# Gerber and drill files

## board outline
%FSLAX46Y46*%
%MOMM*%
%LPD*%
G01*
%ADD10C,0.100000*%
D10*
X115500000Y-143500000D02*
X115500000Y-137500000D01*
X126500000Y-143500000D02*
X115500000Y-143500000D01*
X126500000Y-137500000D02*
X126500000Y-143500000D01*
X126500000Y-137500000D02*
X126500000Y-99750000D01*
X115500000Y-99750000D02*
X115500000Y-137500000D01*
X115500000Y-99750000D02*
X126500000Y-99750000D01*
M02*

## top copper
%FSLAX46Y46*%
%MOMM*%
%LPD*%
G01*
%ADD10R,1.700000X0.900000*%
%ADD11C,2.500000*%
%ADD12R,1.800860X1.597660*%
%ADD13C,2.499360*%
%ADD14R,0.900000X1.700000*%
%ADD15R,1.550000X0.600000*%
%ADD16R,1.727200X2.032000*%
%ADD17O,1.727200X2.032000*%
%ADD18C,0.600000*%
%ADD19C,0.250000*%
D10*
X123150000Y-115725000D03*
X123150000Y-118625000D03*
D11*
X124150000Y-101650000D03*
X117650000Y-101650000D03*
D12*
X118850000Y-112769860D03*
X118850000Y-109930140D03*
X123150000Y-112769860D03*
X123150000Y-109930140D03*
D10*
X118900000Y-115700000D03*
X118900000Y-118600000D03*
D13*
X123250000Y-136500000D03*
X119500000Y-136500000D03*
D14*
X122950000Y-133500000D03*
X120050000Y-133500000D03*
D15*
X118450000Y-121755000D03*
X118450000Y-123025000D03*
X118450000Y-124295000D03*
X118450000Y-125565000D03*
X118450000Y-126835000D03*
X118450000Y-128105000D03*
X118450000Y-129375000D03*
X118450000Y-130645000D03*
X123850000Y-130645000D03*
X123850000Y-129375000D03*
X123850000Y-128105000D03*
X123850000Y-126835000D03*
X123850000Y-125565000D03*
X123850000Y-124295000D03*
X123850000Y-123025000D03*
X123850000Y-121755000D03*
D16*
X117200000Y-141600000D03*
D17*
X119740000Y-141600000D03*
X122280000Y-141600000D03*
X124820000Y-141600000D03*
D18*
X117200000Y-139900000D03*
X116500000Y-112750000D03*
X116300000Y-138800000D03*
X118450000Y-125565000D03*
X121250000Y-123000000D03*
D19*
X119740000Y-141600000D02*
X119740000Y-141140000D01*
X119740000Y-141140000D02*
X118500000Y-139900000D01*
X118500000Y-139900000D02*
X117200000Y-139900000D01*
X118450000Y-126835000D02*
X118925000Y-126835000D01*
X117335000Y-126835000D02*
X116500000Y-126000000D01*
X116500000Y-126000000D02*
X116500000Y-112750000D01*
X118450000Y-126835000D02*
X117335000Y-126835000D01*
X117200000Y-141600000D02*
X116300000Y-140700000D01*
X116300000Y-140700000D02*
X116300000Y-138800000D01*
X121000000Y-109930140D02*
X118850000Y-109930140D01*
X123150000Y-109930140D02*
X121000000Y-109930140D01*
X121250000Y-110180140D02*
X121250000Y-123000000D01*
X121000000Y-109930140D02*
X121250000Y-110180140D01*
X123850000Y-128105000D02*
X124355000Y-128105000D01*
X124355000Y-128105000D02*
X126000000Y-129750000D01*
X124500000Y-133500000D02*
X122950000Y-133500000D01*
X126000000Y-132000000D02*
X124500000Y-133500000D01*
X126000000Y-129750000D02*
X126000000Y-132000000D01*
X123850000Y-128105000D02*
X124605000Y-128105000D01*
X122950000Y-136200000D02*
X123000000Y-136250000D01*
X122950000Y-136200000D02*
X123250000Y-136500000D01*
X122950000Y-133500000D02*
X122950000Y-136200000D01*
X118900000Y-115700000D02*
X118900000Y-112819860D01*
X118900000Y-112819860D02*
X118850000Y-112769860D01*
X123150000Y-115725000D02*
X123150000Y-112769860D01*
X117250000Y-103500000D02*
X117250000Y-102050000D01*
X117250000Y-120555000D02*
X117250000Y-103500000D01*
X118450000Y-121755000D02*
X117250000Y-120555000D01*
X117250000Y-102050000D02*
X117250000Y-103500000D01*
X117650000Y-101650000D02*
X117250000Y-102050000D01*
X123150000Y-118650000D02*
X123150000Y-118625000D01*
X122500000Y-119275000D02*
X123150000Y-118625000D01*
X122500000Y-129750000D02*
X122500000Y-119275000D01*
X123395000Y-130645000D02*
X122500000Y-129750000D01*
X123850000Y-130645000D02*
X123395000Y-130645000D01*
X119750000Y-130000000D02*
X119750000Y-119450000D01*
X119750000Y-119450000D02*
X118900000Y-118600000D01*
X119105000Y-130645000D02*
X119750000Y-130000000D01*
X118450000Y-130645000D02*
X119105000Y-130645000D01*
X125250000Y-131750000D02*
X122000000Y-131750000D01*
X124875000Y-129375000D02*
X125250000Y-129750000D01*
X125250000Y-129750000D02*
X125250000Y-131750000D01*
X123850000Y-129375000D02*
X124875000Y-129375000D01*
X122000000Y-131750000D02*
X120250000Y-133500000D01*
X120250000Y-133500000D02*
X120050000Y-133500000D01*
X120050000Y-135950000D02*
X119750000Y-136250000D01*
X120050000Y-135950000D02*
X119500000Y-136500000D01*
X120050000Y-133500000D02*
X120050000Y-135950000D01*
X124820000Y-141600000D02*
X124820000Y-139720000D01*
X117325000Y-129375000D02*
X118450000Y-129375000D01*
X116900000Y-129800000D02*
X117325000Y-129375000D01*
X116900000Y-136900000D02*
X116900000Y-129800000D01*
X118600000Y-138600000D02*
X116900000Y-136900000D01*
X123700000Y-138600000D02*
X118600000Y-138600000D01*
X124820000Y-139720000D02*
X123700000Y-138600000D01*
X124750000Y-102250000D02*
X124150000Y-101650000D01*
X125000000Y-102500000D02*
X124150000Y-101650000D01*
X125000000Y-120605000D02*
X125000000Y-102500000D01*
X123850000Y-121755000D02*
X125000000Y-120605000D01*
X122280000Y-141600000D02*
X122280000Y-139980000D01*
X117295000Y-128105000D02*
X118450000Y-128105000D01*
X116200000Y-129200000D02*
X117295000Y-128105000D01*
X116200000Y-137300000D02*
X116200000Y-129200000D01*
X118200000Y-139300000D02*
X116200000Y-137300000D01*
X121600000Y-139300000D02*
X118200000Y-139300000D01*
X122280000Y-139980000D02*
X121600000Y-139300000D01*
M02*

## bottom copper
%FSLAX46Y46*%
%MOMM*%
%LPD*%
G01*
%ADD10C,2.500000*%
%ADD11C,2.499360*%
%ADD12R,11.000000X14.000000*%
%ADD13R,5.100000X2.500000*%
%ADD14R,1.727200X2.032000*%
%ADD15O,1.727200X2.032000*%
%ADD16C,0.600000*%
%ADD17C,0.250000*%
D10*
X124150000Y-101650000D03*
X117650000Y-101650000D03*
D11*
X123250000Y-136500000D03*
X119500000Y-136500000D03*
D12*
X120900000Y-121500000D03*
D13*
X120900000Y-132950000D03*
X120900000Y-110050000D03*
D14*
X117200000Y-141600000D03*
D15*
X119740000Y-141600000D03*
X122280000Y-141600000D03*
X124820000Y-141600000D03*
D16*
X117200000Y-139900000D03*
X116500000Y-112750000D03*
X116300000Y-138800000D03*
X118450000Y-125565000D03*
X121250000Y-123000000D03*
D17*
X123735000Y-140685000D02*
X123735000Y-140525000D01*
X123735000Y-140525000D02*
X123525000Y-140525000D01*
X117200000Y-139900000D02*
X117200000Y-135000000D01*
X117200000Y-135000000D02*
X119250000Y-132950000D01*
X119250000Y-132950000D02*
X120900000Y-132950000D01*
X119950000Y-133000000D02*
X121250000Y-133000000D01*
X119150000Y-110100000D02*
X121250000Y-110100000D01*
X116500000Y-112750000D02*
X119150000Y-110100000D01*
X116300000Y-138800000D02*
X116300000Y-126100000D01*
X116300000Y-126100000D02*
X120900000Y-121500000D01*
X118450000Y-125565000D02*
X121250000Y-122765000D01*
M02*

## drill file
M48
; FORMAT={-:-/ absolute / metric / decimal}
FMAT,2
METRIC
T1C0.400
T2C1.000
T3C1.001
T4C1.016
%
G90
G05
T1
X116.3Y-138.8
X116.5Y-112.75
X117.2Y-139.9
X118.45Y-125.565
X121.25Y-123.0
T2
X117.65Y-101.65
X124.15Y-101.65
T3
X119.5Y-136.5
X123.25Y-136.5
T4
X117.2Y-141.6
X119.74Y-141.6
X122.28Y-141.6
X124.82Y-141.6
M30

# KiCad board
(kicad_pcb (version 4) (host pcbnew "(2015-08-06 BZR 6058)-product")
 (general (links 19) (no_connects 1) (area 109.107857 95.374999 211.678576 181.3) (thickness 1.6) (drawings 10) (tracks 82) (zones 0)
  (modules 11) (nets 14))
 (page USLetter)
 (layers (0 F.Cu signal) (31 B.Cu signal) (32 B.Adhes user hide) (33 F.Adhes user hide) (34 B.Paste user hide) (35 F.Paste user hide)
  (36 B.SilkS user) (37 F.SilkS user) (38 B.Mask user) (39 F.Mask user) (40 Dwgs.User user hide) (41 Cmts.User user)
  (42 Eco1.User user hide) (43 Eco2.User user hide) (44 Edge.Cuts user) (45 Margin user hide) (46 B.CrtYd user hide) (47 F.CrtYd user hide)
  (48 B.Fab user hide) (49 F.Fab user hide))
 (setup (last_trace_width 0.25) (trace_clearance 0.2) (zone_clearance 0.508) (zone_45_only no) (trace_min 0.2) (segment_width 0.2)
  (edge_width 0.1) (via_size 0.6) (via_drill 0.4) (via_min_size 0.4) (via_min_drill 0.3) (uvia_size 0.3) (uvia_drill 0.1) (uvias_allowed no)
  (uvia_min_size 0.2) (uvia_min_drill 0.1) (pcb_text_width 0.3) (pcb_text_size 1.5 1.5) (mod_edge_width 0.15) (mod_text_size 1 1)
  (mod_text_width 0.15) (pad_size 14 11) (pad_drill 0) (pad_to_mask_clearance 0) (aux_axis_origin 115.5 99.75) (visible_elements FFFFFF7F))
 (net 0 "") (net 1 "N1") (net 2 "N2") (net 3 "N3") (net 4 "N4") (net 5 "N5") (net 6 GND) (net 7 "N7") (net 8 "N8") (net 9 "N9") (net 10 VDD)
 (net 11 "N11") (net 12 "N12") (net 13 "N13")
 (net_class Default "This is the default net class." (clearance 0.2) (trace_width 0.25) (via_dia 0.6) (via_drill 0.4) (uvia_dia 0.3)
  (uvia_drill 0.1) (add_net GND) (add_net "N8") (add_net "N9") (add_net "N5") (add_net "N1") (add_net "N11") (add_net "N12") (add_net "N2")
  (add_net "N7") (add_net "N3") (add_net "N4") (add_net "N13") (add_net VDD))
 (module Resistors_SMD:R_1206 (layer F.Cu) (at 123.15 117.175 270)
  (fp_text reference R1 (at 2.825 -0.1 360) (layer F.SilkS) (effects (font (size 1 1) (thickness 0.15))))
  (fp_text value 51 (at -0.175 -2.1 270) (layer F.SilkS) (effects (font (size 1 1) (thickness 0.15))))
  (pad 1 smd rect (at -1.45 0 270) (size 0.9 1.7) (layers F.Cu F.Paste F.Mask) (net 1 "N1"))
  (pad 2 smd rect (at 1.45 0 270) (size 0.9 1.7) (layers F.Cu F.Paste F.Mask) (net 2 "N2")))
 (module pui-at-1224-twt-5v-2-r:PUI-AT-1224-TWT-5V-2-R (layer F.Cu) (at 120.9 101.65 180)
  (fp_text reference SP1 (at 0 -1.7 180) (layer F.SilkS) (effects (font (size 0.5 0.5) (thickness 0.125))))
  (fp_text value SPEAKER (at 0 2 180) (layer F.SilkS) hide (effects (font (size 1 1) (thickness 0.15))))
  (pad 1 thru_hole circle (at -3.25 0 180) (size 2.5 2.5) (drill 1) (layers *.Cu *.Mask F.SilkS) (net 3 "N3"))
  (pad 2 thru_hole circle (at 3.25 0 180) (size 2.5 2.5) (drill 1) (layers *.Cu *.Mask F.SilkS) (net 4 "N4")))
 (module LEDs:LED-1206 (layer F.Cu) (at 118.85 111.35 270)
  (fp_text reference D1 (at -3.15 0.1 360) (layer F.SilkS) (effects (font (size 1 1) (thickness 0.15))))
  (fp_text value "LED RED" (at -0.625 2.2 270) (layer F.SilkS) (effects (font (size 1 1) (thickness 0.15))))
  (pad 2 smd rect (at 1.41986 0 90) (size 1.59766 1.80086) (layers F.Cu F.Paste F.Mask) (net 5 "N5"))
  (pad 1 smd rect (at -1.41986 0 90) (size 1.59766 1.80086) (layers F.Cu F.Paste F.Mask) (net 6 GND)))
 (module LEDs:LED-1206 (layer F.Cu) (at 123.15 111.35 270)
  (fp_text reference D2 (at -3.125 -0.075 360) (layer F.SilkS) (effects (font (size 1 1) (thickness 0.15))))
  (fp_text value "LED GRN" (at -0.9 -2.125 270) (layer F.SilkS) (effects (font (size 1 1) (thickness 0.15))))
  (pad 2 smd rect (at 1.41986 0 90) (size 1.59766 1.80086) (layers F.Cu F.Paste F.Mask) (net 1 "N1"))
  (pad 1 smd rect (at -1.41986 0 90) (size 1.59766 1.80086) (layers F.Cu F.Paste F.Mask) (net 6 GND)))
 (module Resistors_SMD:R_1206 (layer F.Cu) (at 118.9 117.15 270)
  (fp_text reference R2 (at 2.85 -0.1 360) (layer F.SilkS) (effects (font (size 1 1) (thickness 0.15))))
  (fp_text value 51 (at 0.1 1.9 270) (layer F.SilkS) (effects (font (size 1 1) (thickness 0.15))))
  (pad 1 smd rect (at -1.45 0 270) (size 0.9 1.7) (layers F.Cu F.Paste F.Mask) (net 5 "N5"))
  (pad 2 smd rect (at 1.45 0 270) (size 0.9 1.7) (layers F.Cu F.Paste F.Mask) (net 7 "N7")))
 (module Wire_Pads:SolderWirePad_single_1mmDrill (layer F.Cu) (at 123.25 136.5)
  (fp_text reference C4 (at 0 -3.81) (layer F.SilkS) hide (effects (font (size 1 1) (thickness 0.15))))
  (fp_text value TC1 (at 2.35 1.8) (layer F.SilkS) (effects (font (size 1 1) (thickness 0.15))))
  (pad 1 thru_hole circle (at 0 0) (size 2.49936 2.49936) (drill 1.00076) (layers *.Cu *.Mask F.SilkS) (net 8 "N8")))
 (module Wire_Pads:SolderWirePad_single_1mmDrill (layer F.Cu) (at 119.5 136.5)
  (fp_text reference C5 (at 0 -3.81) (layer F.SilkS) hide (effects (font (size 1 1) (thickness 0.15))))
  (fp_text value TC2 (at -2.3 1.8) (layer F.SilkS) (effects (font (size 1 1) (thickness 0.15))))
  (pad 1 thru_hole circle (at 0 0) (size 2.49936 2.49936) (drill 1.00076) (layers *.Cu *.Mask F.SilkS) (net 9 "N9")))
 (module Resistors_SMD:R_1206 (layer F.Cu) (at 121.5 133.5 180)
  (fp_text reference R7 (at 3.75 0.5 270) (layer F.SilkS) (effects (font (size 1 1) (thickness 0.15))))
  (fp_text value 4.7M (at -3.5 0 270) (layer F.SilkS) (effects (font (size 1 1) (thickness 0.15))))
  (pad 1 smd rect (at -1.45 0 180) (size 0.9 1.7) (layers F.Cu F.Paste F.Mask) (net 8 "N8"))
  (pad 2 smd rect (at 1.45 0 180) (size 0.9 1.7) (layers F.Cu F.Paste F.Mask) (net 9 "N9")))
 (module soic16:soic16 (layer F.Cu) (at 121.15 126.2) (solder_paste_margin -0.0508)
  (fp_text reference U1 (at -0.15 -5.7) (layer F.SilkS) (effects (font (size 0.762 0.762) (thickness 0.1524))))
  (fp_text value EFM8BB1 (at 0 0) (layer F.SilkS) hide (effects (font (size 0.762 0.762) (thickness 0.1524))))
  (pad 1 smd rect (at -2.7 -4.445) (size 1.55 0.6) (layers F.Cu F.Paste F.Mask) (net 4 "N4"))
  (pad 2 smd rect (at -2.7 -3.175) (size 1.55 0.6) (layers F.Cu F.Paste F.Mask))
  (pad 3 smd rect (at -2.7 -1.905) (size 1.55 0.6) (layers F.Cu F.Paste F.Mask))
  (pad 4 smd rect (at -2.7 -0.635) (size 1.55 0.6) (layers F.Cu F.Paste F.Mask) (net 6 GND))
  (pad 5 smd rect (at -2.7 0.635) (size 1.55 0.6) (layers F.Cu F.Paste F.Mask) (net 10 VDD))
  (pad 6 smd rect (at -2.7 1.905) (size 1.55 0.6) (layers F.Cu F.Paste F.Mask) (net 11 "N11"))
  (pad 7 smd rect (at -2.7 3.175) (size 1.55 0.6) (layers F.Cu F.Paste F.Mask) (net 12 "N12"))
  (pad 8 smd rect (at -2.7 4.445) (size 1.55 0.6) (layers F.Cu F.Paste F.Mask) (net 7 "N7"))
  (pad 9 smd rect (at 2.7 4.445) (size 1.55 0.6) (layers F.Cu F.Paste F.Mask) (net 2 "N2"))
  (pad 10 smd rect (at 2.7 3.175) (size 1.55 0.6) (layers F.Cu F.Paste F.Mask) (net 9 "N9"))
  (pad 11 smd rect (at 2.7 1.905) (size 1.55 0.6) (layers F.Cu F.Paste F.Mask) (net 8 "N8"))
  (pad 12 smd rect (at 2.7 0.635) (size 1.55 0.6) (layers F.Cu F.Paste F.Mask))
  (pad 13 smd rect (at 2.7 -0.635) (size 1.55 0.6) (layers F.Cu F.Paste F.Mask) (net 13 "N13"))
  (pad 14 smd rect (at 2.7 -1.905) (size 1.55 0.6) (layers F.Cu F.Paste F.Mask))
  (pad 15 smd rect (at 2.7 -3.175) (size 1.55 0.6) (layers F.Cu F.Paste F.Mask))
  (pad 16 smd rect (at 2.7 -4.445) (size 1.55 0.6) (layers F.Cu F.Paste F.Mask) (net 3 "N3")))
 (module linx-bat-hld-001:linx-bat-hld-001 (layer B.Cu) (at 120.9 121.5 90)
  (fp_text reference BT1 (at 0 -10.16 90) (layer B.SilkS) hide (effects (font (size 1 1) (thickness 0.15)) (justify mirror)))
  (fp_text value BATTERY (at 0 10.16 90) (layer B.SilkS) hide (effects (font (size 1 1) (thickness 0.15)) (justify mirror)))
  (pad 2 smd rect (at 0 0 90) (size 14 11) (layers B.Cu B.Paste B.Mask) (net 6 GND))
  (pad 1 smd rect (at -11.45 0 90) (size 2.5 5.1) (layers B.Cu B.Paste B.Mask) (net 10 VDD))
  (pad 1 smd rect (at 11.45 0 90) (size 2.5 5.1) (layers B.Cu B.Paste B.Mask) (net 10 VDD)))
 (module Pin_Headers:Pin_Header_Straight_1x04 (layer F.Cu) (at 117.2 141.6 90)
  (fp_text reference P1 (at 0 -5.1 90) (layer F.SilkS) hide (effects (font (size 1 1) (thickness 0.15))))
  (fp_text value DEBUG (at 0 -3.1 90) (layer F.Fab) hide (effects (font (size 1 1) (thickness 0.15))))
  (pad 1 thru_hole rect (at 0 0 90) (size 2.032 1.7272) (drill 1.016) (layers *.Cu *.Mask F.SilkS) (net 6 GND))
  (pad 2 thru_hole oval (at 0 2.54 90) (size 2.032 1.7272) (drill 1.016) (layers *.Cu *.Mask F.SilkS) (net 10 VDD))
  (pad 3 thru_hole oval (at 0 5.08 90) (size 2.032 1.7272) (drill 1.016) (layers *.Cu *.Mask F.SilkS) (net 11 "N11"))
  (pad 4 thru_hole oval (at 0 7.62 90) (size 2.032 1.7272) (drill 1.016) (layers *.Cu *.Mask F.SilkS) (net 12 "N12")))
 (gr_line (start 115.5 143.5) (end 115.5 137.5) (angle 90) (layer Edge.Cuts) (width 0.1))
 (gr_line (start 126.5 143.5) (end 115.5 143.5) (angle 90) (layer Edge.Cuts) (width 0.1))
 (gr_line (start 126.5 137.5) (end 126.5 143.5) (angle 90) (layer Edge.Cuts) (width 0.1))
 (gr_line (start 126.5 137.5) (end 126.5 99.75) (angle 90) (layer Edge.Cuts) (width 0.1))
 (gr_line (start 115.5 99.75) (end 115.5 137.5) (angle 90) (layer Edge.Cuts) (width 0.1))
 (gr_line (start 115.5 99.75) (end 126.5 99.75) (angle 90) (layer Edge.Cuts) (width 0.1))
 (segment (start 123.735 140.685) (end 123.735 140.525) (width 0.25) (layer B.Cu) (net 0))
 (segment (start 123.735 140.525) (end 123.525 140.525) (width 0.25) (layer B.Cu) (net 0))
 (segment (start 119.74 141.6) (end 119.74 141.14) (width 0.25) (layer F.Cu) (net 10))
 (segment (start 119.74 141.14) (end 118.5 139.9) (width 0.25) (layer F.Cu) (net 10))
 (segment (start 118.5 139.9) (end 117.2 139.9) (width 0.25) (layer F.Cu) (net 10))
 (via (at 117.2 139.9) (size 0.6) (drill 0.4) (layers F.Cu B.Cu) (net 10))
 (segment (start 117.2 139.9) (end 117.2 135) (width 0.25) (layer B.Cu) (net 10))
 (segment (start 117.2 135) (end 119.25 132.95) (width 0.25) (layer B.Cu) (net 10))
 (segment (start 119.25 132.95) (end 120.9 132.95) (width 0.25) (layer B.Cu) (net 10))
 (segment (start 119.95 133) (end 121.25 133) (width 0.25) (layer B.Cu) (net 10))
 (segment (start 118.45 126.835) (end 118.925 126.835) (width 0.25) (layer F.Cu) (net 10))
 (segment (start 119.15 110.1) (end 121.25 110.1) (width 0.25) (layer B.Cu) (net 10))
 (segment (start 117.335 126.835) (end 116.5 126) (width 0.25) (layer F.Cu) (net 10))
 (segment (start 116.5 126) (end 116.5 112.75) (width 0.25) (layer F.Cu) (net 10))
 (via (at 116.5 112.75) (size 0.6) (layers F.Cu B.Cu) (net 10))
 (segment (start 116.5 112.75) (end 119.15 110.1) (width 0.25) (layer B.Cu) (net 10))
 (segment (start 118.45 126.835) (end 117.335 126.835) (width 0.25) (layer F.Cu) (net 10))
 (segment (start 117.2 141.6) (end 116.3 140.7) (width 0.25) (layer F.Cu) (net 6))
 (segment (start 116.3 138.8) (end 116.3 126.1) (width 0.25) (layer B.Cu) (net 6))
 (via (at 116.3 138.8) (size 0.6) (drill 0.4) (layers F.Cu B.Cu) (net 6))
 (segment (start 116.3 140.7) (end 116.3 138.8) (width 0.25) (layer F.Cu) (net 6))
 (segment (start 116.3 126.1) (end 120.9 121.5) (width 0.25) (layer B.Cu) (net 6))
 (segment (start 118.45 125.565) (end 121.25 122.765) (width 0.25) (layer B.Cu) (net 6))
 (via (at 118.45 125.565) (size 0.6) (layers F.Cu B.Cu) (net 6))
 (segment (start 121 109.93014) (end 118.85 109.93014) (width 0.25) (layer F.Cu) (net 6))
 (segment (start 123.15 109.93014) (end 121 109.93014) (width 0.25) (layer F.Cu) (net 6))
 (segment (start 121.25 110.18014) (end 121.25 123) (width 0.25) (layer F.Cu) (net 6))
 (via (at 121.25 123) (size 0.6) (layers F.Cu B.Cu) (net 6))
 (segment (start 121 109.93014) (end 121.25 110.18014) (width 0.25) (layer F.Cu) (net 6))
 (segment (start 123.85 128.105) (end 124.355 128.105) (width 0.25) (layer F.Cu) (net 8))
 (segment (start 124.355 128.105) (end 126 129.75) (width 0.25) (layer F.Cu) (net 8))
 (segment (start 124.5 133.5) (end 122.95 133.5) (width 0.25) (layer F.Cu) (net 8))
 (segment (start 126 132) (end 124.5 133.5) (width 0.25) (layer F.Cu) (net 8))
 (segment (start 126 129.75) (end 126 132) (width 0.25) (layer F.Cu) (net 8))
 (segment (start 123.85 128.105) (end 124.605 128.105) (width 0.25) (layer F.Cu) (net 8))
 (segment (start 122.95 136.2) (end 123 136.25) (width 0.25) (layer F.Cu) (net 8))
 (segment (start 122.95 136.2) (end 123.25 136.5) (width 0.25) (layer F.Cu) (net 8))
 (segment (start 122.95 133.5) (end 122.95 136.2) (width 0.25) (layer F.Cu) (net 8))
 (segment (start 118.9 115.7) (end 118.9 112.81986) (width 0.25) (layer F.Cu) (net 5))
 (segment (start 118.9 112.81986) (end 118.85 112.76986) (width 0.25) (layer F.Cu) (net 5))
 (segment (start 123.15 115.725) (end 123.15 112.76986) (width 0.25) (layer F.Cu) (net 1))
 (segment (start 117.25 103.5) (end 117.25 102.05) (width 0.25) (layer F.Cu) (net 4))
 (segment (start 117.25 120.555) (end 117.25 103.5) (width 0.25) (layer F.Cu) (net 4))
 (segment (start 118.45 121.755) (end 117.25 120.555) (width 0.25) (layer F.Cu) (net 4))
 (segment (start 117.25 102.05) (end 117.25 103.5) (width 0.25) (layer F.Cu) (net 4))
 (segment (start 117.65 101.65) (end 117.25 102.05) (width 0.25) (layer F.Cu) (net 4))
 (segment (start 123.15 118.65) (end 123.15 118.625) (width 0.25) (layer F.Cu) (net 2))
 (segment (start 122.5 119.275) (end 123.15 118.625) (width 0.25) (layer F.Cu) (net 2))
 (segment (start 122.5 129.75) (end 122.5 119.275) (width 0.25) (layer F.Cu) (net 2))
 (segment (start 123.395 130.645) (end 122.5 129.75) (width 0.25) (layer F.Cu) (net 2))
 (segment (start 123.85 130.645) (end 123.395 130.645) (width 0.25) (layer F.Cu) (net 2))
 (segment (start 119.75 130) (end 119.75 119.45) (width 0.25) (layer F.Cu) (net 7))
 (segment (start 119.75 119.45) (end 118.9 118.6) (width 0.25) (layer F.Cu) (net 7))
 (segment (start 119.105 130.645) (end 119.75 130) (width 0.25) (layer F.Cu) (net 7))
 (segment (start 118.45 130.645) (end 119.105 130.645) (width 0.25) (layer F.Cu) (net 7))
 (segment (start 125.25 131.75) (end 122 131.75) (width 0.25) (layer F.Cu) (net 9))
 (segment (start 124.875 129.375) (end 125.25 129.75) (width 0.25) (layer F.Cu) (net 9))
 (segment (start 125.25 129.75) (end 125.25 131.75) (width 0.25) (layer F.Cu) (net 9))
 (segment (start 123.85 129.375) (end 124.875 129.375) (width 0.25) (layer F.Cu) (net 9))
 (segment (start 122 131.75) (end 120.25 133.5) (width 0.25) (layer F.Cu) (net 9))
 (segment (start 120.25 133.5) (end 120.05 133.5) (width 0.25) (layer F.Cu) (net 9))
 (segment (start 120.05 135.95) (end 119.75 136.25) (width 0.25) (layer F.Cu) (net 9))
 (segment (start 120.05 135.95) (end 119.5 136.5) (width 0.25) (layer F.Cu) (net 9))
 (segment (start 120.05 133.5) (end 120.05 135.95) (width 0.25) (layer F.Cu) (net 9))
 (segment (start 124.82 141.6) (end 124.82 139.72) (width 0.25) (layer F.Cu) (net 12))
 (segment (start 117.325 129.375) (end 118.45 129.375) (width 0.25) (layer F.Cu) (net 12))
 (segment (start 116.9 129.8) (end 117.325 129.375) (width 0.25) (layer F.Cu) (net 12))
 (segment (start 116.9 136.9) (end 116.9 129.8) (width 0.25) (layer F.Cu) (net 12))
 (segment (start 118.6 138.6) (end 116.9 136.9) (width 0.25) (layer F.Cu) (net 12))
 (segment (start 123.7 138.6) (end 118.6 138.6) (width 0.25) (layer F.Cu) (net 12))
 (segment (start 124.82 139.72) (end 123.7 138.6) (width 0.25) (layer F.Cu) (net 12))
 (segment (start 124.75 102.25) (end 124.15 101.65) (width 0.25) (layer F.Cu) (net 3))
 (segment (start 125 102.5) (end 124.15 101.65) (width 0.25) (layer F.Cu) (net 3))
 (segment (start 125 120.605) (end 125 102.5) (width 0.25) (layer F.Cu) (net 3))
 (segment (start 123.85 121.755) (end 125 120.605) (width 0.25) (layer F.Cu) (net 3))
 (segment (start 122.28 141.6) (end 122.28 139.98) (width 0.25) (layer F.Cu) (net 11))
 (segment (start 117.295 128.105) (end 118.45 128.105) (width 0.25) (layer F.Cu) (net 11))
 (segment (start 116.2 129.2) (end 117.295 128.105) (width 0.25) (layer F.Cu) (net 11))
 (segment (start 116.2 137.3) (end 116.2 129.2) (width 0.25) (layer F.Cu) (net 11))
 (segment (start 118.2 139.3) (end 116.2 137.3) (width 0.25) (layer F.Cu) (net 11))
 (segment (start 121.6 139.3) (end 118.2 139.3) (width 0.25) (layer F.Cu) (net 11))
 (segment (start 122.28 139.98) (end 121.6 139.3) (width 0.25) (layer F.Cu) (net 11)))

